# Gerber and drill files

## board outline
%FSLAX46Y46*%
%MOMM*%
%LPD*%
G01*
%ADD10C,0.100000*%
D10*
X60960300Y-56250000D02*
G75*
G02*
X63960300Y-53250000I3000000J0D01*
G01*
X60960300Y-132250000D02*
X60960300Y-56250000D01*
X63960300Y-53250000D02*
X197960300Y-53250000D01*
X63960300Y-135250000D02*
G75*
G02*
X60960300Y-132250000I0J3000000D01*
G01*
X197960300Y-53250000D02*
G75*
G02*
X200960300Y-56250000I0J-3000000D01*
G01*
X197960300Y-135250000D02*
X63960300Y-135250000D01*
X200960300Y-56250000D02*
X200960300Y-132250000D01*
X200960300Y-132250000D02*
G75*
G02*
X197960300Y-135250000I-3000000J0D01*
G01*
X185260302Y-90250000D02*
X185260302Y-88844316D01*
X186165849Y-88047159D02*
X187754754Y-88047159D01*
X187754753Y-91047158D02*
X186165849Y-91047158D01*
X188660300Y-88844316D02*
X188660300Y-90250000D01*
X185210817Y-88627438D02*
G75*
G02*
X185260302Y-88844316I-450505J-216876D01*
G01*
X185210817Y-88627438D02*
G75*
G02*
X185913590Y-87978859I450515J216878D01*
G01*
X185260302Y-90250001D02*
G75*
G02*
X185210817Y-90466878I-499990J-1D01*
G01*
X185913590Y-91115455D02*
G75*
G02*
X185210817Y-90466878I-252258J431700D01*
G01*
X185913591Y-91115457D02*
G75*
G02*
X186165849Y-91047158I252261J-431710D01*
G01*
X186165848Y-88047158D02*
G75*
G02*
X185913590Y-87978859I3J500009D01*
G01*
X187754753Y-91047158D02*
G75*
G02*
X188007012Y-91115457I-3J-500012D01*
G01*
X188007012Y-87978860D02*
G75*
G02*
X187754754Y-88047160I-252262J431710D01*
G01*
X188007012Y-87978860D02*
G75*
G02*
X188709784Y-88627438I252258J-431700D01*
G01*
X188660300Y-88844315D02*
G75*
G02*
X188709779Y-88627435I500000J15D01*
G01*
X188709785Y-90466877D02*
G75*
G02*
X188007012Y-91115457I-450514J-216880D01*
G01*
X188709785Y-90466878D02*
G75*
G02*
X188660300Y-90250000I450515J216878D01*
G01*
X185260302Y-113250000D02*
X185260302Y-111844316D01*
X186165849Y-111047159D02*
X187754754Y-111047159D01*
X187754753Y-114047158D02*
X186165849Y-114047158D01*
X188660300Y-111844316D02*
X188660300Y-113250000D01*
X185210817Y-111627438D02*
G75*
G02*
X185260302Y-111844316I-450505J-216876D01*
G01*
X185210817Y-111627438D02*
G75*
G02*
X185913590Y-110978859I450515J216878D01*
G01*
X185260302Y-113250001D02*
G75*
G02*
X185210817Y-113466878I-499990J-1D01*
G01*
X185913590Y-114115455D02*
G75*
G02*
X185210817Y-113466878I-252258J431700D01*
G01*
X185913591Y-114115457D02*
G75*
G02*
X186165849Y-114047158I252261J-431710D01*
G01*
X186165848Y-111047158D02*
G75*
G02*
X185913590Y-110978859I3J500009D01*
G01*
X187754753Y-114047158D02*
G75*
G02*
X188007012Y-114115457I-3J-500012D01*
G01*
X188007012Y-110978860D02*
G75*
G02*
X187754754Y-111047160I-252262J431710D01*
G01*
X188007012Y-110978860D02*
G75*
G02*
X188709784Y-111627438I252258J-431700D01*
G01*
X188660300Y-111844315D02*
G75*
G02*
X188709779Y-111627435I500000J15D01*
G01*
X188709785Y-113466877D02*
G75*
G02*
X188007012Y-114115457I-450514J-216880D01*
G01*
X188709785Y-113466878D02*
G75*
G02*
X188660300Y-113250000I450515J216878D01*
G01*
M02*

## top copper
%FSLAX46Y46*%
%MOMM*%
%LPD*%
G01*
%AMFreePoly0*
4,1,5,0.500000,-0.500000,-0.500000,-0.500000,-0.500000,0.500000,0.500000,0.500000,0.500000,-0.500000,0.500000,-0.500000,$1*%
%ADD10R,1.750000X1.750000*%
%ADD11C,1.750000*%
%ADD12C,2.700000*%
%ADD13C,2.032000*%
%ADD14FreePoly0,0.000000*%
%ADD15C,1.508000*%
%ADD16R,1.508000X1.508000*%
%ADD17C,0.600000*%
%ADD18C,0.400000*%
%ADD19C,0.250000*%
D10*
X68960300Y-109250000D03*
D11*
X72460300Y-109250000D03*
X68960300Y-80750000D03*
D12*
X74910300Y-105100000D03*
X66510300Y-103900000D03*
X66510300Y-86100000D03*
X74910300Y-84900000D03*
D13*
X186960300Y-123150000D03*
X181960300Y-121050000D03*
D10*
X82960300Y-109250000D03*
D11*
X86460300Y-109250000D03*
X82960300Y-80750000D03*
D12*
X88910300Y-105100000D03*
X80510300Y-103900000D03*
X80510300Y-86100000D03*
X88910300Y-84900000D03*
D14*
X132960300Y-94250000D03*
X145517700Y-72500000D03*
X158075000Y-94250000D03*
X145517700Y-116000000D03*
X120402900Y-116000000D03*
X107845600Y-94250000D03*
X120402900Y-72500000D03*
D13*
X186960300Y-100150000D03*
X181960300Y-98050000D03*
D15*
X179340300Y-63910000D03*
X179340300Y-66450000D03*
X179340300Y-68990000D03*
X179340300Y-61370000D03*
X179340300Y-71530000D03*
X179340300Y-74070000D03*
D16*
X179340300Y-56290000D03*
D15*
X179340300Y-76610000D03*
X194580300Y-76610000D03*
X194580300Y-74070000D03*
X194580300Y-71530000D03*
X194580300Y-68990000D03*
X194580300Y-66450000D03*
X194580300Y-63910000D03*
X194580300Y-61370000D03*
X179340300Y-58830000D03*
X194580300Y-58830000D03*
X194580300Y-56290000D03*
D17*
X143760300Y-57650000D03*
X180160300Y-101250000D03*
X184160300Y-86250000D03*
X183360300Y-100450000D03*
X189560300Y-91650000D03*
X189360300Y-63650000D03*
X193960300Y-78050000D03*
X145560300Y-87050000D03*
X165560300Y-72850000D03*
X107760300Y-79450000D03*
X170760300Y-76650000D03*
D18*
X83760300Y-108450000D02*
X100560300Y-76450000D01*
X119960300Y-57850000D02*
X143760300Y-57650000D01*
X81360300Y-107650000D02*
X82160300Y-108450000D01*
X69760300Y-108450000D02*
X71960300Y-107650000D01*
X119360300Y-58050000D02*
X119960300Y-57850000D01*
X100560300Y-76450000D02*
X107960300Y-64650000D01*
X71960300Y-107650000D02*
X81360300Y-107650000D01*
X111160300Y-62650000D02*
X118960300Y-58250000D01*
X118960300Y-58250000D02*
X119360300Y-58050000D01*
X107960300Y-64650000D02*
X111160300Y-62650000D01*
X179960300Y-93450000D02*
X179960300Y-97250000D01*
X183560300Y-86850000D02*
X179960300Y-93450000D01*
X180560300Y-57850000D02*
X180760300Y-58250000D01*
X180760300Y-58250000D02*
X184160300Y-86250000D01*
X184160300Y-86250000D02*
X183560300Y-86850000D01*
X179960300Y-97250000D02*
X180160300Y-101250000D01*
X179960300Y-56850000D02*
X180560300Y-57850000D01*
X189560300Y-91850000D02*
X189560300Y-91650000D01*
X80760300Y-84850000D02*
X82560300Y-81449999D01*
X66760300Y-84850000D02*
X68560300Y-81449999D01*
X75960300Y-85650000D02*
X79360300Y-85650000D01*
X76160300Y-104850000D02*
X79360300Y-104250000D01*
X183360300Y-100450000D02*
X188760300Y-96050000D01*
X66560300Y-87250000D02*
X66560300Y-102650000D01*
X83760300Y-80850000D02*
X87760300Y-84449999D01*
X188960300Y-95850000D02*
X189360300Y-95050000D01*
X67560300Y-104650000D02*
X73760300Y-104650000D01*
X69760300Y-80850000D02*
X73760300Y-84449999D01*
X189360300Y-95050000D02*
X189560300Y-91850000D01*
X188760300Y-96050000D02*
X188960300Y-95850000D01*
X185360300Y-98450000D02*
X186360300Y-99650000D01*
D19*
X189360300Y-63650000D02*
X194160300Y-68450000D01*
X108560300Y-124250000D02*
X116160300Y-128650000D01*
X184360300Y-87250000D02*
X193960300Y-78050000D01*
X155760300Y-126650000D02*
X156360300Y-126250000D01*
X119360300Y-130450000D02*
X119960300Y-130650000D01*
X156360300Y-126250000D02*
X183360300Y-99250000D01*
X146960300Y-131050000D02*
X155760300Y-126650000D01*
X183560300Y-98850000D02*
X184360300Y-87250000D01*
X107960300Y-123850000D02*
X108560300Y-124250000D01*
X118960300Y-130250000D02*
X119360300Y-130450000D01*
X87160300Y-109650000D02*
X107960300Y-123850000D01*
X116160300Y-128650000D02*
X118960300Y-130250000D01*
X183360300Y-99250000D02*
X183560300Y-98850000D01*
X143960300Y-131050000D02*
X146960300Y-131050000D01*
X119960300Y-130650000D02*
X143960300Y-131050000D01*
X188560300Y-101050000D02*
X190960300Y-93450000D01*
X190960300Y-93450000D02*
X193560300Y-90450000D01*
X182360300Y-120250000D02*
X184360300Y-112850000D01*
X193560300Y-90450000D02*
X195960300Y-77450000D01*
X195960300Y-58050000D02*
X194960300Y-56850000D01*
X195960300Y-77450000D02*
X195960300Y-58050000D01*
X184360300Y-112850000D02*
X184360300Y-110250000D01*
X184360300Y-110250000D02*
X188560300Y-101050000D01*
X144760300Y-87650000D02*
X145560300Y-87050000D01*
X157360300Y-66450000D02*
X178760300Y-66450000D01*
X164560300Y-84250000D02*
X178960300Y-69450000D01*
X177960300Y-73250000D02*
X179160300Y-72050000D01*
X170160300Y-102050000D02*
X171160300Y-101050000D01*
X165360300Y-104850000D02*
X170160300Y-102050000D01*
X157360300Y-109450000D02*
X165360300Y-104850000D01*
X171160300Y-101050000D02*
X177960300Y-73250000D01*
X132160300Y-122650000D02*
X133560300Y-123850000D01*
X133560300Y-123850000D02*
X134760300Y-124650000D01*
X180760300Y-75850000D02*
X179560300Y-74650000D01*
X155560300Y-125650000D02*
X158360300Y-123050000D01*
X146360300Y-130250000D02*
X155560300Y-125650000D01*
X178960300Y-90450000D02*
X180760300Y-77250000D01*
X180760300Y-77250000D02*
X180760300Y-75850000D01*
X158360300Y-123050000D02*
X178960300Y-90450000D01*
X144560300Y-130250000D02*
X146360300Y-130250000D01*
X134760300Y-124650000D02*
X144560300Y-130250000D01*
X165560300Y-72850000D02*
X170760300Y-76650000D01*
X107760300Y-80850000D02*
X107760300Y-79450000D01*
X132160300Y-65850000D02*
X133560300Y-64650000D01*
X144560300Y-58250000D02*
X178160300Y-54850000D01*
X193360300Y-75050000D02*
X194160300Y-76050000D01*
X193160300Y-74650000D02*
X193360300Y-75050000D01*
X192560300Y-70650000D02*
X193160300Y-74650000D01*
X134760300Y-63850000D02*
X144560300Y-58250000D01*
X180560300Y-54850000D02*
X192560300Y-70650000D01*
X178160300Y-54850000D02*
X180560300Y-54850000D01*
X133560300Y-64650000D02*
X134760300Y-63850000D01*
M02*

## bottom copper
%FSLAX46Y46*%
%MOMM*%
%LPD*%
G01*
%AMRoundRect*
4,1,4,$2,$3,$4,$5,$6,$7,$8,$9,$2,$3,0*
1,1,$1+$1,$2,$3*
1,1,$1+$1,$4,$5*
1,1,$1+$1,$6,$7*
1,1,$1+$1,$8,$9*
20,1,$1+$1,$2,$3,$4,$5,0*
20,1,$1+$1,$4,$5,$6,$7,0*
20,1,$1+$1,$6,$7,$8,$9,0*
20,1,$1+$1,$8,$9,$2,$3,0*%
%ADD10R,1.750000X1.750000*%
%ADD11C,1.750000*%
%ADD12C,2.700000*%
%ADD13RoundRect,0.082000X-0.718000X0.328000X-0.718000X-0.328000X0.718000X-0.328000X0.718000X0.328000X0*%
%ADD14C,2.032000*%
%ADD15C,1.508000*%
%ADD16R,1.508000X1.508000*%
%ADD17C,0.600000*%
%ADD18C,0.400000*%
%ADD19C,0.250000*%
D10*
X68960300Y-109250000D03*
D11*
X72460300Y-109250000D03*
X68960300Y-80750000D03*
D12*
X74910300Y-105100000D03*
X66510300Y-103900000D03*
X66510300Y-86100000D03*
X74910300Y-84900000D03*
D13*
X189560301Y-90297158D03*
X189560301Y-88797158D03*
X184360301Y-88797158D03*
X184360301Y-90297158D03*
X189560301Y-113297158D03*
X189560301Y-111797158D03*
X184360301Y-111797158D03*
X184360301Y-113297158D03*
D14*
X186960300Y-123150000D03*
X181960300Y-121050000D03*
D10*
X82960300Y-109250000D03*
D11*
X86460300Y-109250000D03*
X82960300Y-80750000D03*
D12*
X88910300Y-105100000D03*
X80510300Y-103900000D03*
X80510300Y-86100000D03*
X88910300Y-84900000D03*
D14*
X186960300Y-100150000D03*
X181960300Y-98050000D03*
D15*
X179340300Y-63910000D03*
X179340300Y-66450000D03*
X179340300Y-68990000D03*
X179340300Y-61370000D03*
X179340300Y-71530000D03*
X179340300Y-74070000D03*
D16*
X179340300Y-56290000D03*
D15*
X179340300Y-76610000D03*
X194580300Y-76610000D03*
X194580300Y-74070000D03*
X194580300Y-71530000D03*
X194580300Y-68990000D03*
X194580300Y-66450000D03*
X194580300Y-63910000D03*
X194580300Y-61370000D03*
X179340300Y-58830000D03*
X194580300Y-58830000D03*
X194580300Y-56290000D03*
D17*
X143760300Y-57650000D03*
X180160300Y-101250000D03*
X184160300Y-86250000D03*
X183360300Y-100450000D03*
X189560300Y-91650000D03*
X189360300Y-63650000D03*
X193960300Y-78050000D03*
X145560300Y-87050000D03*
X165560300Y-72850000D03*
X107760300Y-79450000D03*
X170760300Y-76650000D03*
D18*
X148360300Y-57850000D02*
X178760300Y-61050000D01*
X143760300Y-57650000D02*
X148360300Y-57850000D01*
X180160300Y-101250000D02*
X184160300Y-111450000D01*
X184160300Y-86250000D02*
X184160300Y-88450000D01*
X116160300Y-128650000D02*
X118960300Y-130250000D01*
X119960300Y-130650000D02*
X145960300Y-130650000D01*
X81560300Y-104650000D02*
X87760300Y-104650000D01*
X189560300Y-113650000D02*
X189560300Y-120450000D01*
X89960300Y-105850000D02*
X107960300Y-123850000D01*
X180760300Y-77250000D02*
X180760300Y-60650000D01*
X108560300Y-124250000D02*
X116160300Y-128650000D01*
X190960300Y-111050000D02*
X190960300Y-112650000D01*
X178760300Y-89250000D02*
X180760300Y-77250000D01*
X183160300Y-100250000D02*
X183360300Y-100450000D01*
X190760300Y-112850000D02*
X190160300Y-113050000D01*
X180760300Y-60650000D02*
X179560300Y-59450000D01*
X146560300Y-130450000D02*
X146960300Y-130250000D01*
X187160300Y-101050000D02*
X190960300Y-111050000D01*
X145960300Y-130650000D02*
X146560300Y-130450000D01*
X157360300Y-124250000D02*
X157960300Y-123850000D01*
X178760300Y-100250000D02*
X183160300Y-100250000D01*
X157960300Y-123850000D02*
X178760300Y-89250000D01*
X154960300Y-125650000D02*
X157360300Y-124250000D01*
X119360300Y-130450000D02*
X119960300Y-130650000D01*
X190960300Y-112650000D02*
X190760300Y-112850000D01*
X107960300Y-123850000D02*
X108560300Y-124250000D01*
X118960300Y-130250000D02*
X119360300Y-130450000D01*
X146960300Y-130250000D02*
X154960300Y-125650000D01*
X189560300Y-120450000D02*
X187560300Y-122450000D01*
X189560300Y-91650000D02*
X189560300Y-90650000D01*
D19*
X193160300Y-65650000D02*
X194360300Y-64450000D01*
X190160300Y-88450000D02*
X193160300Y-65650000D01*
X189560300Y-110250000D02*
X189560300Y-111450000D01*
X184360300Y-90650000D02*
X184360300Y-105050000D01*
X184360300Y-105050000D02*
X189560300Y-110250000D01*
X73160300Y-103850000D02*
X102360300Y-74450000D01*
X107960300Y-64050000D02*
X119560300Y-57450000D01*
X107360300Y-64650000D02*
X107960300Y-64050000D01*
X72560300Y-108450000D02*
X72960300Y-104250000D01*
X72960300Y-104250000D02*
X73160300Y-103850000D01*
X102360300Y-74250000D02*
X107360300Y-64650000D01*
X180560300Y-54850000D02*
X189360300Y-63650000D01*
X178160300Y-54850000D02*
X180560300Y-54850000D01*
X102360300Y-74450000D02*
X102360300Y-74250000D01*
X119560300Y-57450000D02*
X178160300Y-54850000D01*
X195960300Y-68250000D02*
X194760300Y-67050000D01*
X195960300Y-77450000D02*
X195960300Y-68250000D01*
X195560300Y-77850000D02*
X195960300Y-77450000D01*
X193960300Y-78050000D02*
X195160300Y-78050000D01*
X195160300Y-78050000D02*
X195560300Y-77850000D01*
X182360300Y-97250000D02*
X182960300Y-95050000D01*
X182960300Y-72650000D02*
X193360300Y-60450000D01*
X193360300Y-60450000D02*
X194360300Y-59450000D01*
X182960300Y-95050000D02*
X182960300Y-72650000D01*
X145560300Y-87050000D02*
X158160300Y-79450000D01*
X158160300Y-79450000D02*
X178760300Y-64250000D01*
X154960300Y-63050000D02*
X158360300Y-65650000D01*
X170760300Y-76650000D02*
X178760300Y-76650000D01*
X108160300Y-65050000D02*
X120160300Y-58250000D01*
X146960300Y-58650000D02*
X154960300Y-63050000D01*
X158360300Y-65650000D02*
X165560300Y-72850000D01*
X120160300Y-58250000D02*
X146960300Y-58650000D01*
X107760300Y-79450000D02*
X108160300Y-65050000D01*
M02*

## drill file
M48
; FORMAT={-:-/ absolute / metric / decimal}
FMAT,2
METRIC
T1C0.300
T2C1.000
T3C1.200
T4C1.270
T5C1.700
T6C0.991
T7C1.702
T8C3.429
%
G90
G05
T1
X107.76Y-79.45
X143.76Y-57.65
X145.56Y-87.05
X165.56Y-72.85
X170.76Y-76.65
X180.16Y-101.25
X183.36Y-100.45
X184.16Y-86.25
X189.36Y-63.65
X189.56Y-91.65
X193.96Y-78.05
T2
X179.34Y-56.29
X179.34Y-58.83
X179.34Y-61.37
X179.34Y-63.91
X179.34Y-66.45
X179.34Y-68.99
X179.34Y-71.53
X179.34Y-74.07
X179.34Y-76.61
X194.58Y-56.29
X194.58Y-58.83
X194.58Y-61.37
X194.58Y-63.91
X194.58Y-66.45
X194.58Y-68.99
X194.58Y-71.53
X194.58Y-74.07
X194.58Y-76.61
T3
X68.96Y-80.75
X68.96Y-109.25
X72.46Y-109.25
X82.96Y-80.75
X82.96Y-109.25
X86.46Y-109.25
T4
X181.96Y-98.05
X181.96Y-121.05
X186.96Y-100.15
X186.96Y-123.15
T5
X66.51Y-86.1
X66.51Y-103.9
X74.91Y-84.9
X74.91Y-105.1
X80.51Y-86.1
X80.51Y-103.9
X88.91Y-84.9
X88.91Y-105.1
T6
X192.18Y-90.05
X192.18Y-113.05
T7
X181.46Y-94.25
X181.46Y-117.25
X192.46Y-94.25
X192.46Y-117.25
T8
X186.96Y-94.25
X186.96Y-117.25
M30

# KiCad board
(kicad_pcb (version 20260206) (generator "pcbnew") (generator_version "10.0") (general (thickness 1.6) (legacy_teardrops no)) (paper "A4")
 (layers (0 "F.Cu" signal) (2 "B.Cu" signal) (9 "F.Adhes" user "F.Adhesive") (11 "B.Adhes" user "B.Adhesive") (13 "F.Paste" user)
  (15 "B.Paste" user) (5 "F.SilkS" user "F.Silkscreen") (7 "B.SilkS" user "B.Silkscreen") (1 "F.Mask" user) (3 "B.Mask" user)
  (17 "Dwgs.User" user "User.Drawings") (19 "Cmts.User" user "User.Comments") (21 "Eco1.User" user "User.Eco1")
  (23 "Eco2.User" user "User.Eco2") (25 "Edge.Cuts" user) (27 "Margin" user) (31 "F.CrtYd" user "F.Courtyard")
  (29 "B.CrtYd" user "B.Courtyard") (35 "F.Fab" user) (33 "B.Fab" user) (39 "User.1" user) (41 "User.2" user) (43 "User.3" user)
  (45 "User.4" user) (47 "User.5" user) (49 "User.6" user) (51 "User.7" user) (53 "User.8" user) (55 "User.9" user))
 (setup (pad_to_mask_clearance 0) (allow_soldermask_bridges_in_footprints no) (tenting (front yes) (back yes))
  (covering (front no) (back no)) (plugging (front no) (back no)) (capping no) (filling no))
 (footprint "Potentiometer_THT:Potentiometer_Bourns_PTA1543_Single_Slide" (layer "F.Cu") (at 68.9603 109.25 90)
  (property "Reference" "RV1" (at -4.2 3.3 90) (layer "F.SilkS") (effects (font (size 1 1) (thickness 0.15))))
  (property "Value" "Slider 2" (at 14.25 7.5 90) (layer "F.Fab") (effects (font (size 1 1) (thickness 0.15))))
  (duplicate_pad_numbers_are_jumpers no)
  (pad "1" thru_hole rect (at 0 0 90) (size 1.75 1.75) (drill 1.2) (layers "*.Cu" "*.Mask") (remove_unused_layers no) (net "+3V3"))
  (pad "2" thru_hole circle (at 0 3.5 90) (size 1.75 1.75) (drill 1.2) (layers "*.Cu" "*.Mask") (remove_unused_layers no) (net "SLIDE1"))
  (pad "3" thru_hole circle (at 28.5 0 90) (size 1.75 1.75) (drill 1.2) (layers "*.Cu" "*.Mask") (remove_unused_layers no) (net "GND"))
  (pad "MP" thru_hole circle (at 4.15 5.95 90) (size 2.7 2.7) (drill 1.7) (layers "*.Cu" "*.Mask") (remove_unused_layers no) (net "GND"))
  (pad "MP" thru_hole circle (at 5.35 -2.45 90) (size 2.7 2.7) (drill 1.7) (layers "*.Cu" "*.Mask") (remove_unused_layers no) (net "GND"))
  (pad "MP" thru_hole circle (at 23.15 -2.45 90) (size 2.7 2.7) (drill 1.7) (layers "*.Cu" "*.Mask") (remove_unused_layers no) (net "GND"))
  (pad "MP" thru_hole circle (at 24.35 5.95 90) (size 2.7 2.7) (drill 1.7) (layers "*.Cu" "*.Mask") (remove_unused_layers no) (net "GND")))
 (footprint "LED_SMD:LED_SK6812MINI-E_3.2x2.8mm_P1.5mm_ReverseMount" (layer "F.Cu") (at 186.9603 89.65)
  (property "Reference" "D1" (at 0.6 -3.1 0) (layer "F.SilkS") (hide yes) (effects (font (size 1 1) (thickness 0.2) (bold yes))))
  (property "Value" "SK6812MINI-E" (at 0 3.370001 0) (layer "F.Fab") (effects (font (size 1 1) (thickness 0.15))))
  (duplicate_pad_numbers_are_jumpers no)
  (fp_line (start -1.699998 0.6) (end -1.699998 -0.805684) (stroke (width 0.1) (type solid)) (layer "Edge.Cuts"))
  (fp_line (start -0.794451 -1.602841) (end 0.794454 -1.602841) (stroke (width 0.1) (type solid)) (layer "Edge.Cuts"))
  (fp_line (start 0.794453 1.397158) (end -0.794451 1.397158) (stroke (width 0.1) (type solid)) (layer "Edge.Cuts"))
  (fp_line (start 1.7 -0.805684) (end 1.7 0.6) (stroke (width 0.1) (type solid)) (layer "Edge.Cuts"))
  (fp_arc (start -1.749483 -1.022562) (mid -1.712526 -0.91691) (end -1.699998 -0.805684) (stroke (width 0.1) (type solid))
   (layer "Edge.Cuts"))
  (fp_arc (start -1.749483 -1.022562) (mid -1.63807 -1.606877) (end -1.04671 -1.671141) (stroke (width 0.1) (type solid))
   (layer "Edge.Cuts"))
  (fp_arc (start -1.699998 0.600001) (mid -1.712526 0.711226) (end -1.749483 0.816878) (stroke (width 0.1) (type solid)) (layer "Edge.Cuts"))
  (fp_arc (start -1.04671 1.465455) (mid -1.638069 1.401192) (end -1.749483 0.816878) (stroke (width 0.1) (type solid)) (layer "Edge.Cuts"))
  (fp_arc (start -1.046709 1.465457) (mid -0.925121 1.414535) (end -0.794451 1.397158) (stroke (width 0.1) (type solid)) (layer "Edge.Cuts"))
  (fp_arc (start -0.794452 -1.602842) (mid -0.925122 -1.620219) (end -1.04671 -1.671141) (stroke (width 0.1) (type solid))
   (layer "Edge.Cuts"))
  (fp_arc (start 0.794453 1.397158) (mid 0.925124 1.414535) (end 1.046712 1.465457) (stroke (width 0.1) (type solid)) (layer "Edge.Cuts"))
  (fp_arc (start 1.046712 -1.67114) (mid 0.925124 -1.620218) (end 0.794454 -1.602841) (stroke (width 0.1) (type solid)) (layer "Edge.Cuts"))
  (fp_arc (start 1.046712 -1.67114) (mid 1.638072 -1.606876) (end 1.749485 -1.022562) (stroke (width 0.1) (type solid)) (layer "Edge.Cuts"))
  (fp_arc (start 1.7 -0.805685) (mid 1.712528 -0.91691) (end 1.749485 -1.022562) (stroke (width 0.1) (type solid)) (layer "Edge.Cuts"))
  (fp_arc (start 1.749485 0.816877) (mid 1.638073 1.401193) (end 1.046712 1.465457) (stroke (width 0.1) (type solid)) (layer "Edge.Cuts"))
  (fp_arc (start 1.749485 0.816878) (mid 1.712528 0.711226) (end 1.7 0.6) (stroke (width 0.1) (type solid)) (layer "Edge.Cuts"))
  (pad "1" smd roundrect (at 2.600001 0.647158 270) (size 0.82 1.6) (layers "B.Cu" "B.Mask" "B.Paste") (roundrect_rratio 0.1) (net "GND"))
  (pad "2" smd roundrect (at 2.600001 -0.852842 270) (size 0.82 1.6) (layers "B.Cu" "B.Mask" "B.Paste") (roundrect_rratio 0.1) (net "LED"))
  (pad "3" smd roundrect (at -2.599999 -0.852842 270) (size 0.82 1.6) (layers "B.Cu" "B.Mask" "B.Paste") (roundrect_rratio 0.1) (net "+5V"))
  (pad "4" smd roundrect (at -2.599999 0.647158 270) (size 0.82 1.6) (layers "B.Cu" "B.Mask" "B.Paste") (roundrect_rratio 0.1)
   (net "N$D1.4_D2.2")))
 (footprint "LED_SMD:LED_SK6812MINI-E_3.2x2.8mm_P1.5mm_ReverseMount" (layer "F.Cu") (at 186.9603 112.65)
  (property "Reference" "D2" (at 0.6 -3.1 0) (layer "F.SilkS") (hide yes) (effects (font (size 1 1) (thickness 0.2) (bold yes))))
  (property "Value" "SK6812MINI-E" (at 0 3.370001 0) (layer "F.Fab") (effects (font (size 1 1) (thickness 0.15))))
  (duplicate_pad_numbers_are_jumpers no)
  (fp_line (start -1.699998 0.6) (end -1.699998 -0.805684) (stroke (width 0.1) (type solid)) (layer "Edge.Cuts"))
  (fp_line (start -0.794451 -1.602841) (end 0.794454 -1.602841) (stroke (width 0.1) (type solid)) (layer "Edge.Cuts"))
  (fp_line (start 0.794453 1.397158) (end -0.794451 1.397158) (stroke (width 0.1) (type solid)) (layer "Edge.Cuts"))
  (fp_line (start 1.7 -0.805684) (end 1.7 0.6) (stroke (width 0.1) (type solid)) (layer "Edge.Cuts"))
  (fp_arc (start -1.749483 -1.022562) (mid -1.712526 -0.91691) (end -1.699998 -0.805684) (stroke (width 0.1) (type solid))
   (layer "Edge.Cuts"))
  (fp_arc (start -1.749483 -1.022562) (mid -1.63807 -1.606877) (end -1.04671 -1.671141) (stroke (width 0.1) (type solid))
   (layer "Edge.Cuts"))
  (fp_arc (start -1.699998 0.600001) (mid -1.712526 0.711226) (end -1.749483 0.816878) (stroke (width 0.1) (type solid)) (layer "Edge.Cuts"))
  (fp_arc (start -1.04671 1.465455) (mid -1.638069 1.401192) (end -1.749483 0.816878) (stroke (width 0.1) (type solid)) (layer "Edge.Cuts"))
  (fp_arc (start -1.046709 1.465457) (mid -0.925121 1.414535) (end -0.794451 1.397158) (stroke (width 0.1) (type solid)) (layer "Edge.Cuts"))
  (fp_arc (start -0.794452 -1.602842) (mid -0.925122 -1.620219) (end -1.04671 -1.671141) (stroke (width 0.1) (type solid))
   (layer "Edge.Cuts"))
  (fp_arc (start 0.794453 1.397158) (mid 0.925124 1.414535) (end 1.046712 1.465457) (stroke (width 0.1) (type solid)) (layer "Edge.Cuts"))
  (fp_arc (start 1.046712 -1.67114) (mid 0.925124 -1.620218) (end 0.794454 -1.602841) (stroke (width 0.1) (type solid)) (layer "Edge.Cuts"))
  (fp_arc (start 1.046712 -1.67114) (mid 1.638072 -1.606876) (end 1.749485 -1.022562) (stroke (width 0.1) (type solid)) (layer "Edge.Cuts"))
  (fp_arc (start 1.7 -0.805685) (mid 1.712528 -0.91691) (end 1.749485 -1.022562) (stroke (width 0.1) (type solid)) (layer "Edge.Cuts"))
  (fp_arc (start 1.749485 0.816877) (mid 1.638073 1.401193) (end 1.046712 1.465457) (stroke (width 0.1) (type solid)) (layer "Edge.Cuts"))
  (fp_arc (start 1.749485 0.816878) (mid 1.712528 0.711226) (end 1.7 0.6) (stroke (width 0.1) (type solid)) (layer "Edge.Cuts"))
  (pad "1" smd roundrect (at 2.600001 0.647158 270) (size 0.82 1.6) (layers "B.Cu" "B.Mask" "B.Paste") (roundrect_rratio 0.1) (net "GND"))
  (pad "2" smd roundrect (at 2.600001 -0.852842 270) (size 0.82 1.6) (layers "B.Cu" "B.Mask" "B.Paste") (roundrect_rratio 0.1)
   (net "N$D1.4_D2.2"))
  (pad "3" smd roundrect (at -2.599999 -0.852842 270) (size 0.82 1.6) (layers "B.Cu" "B.Mask" "B.Paste") (roundrect_rratio 0.1) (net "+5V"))
  (pad "4" smd roundrect (at -2.599999 0.647158 270) (size 0.82 1.6) (layers "B.Cu" "B.Mask" "B.Paste") (roundrect_rratio 0.1)))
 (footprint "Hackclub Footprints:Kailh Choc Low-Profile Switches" (layer "F.Cu") (at 186.9603 117.25)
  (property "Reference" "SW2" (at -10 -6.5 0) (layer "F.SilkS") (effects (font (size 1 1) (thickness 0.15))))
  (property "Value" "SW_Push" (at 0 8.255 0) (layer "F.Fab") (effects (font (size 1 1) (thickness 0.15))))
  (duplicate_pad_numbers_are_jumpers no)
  (pad "" np_thru_hole circle (at -5.5 0) (size 1.7018 1.7018) (drill 1.7018) (layers "*.Cu" "*.Mask"))
  (pad "" np_thru_hole circle (at 0 0) (size 3.429 3.429) (drill 3.429) (layers "*.Cu" "*.Mask"))
  (pad "" np_thru_hole circle (at 5.22 -4.2) (size 0.9906 0.9906) (drill 0.9906) (layers "*.Cu" "*.Mask"))
  (pad "" np_thru_hole circle (at 5.5 0) (size 1.7018 1.7018) (drill 1.7018) (layers "*.Cu" "*.Mask"))
  (pad "1" thru_hole circle (at 0 5.9) (size 2.032 2.032) (drill 1.27) (layers "*.Cu" "*.Mask") (remove_unused_layers no) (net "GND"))
  (pad "2" thru_hole circle (at -5 3.8) (size 2.032 2.032) (drill 1.27) (layers "*.Cu" "*.Mask") (remove_unused_layers no) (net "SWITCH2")))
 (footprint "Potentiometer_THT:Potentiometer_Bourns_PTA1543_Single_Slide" (layer "F.Cu") (at 82.9603 109.25 90)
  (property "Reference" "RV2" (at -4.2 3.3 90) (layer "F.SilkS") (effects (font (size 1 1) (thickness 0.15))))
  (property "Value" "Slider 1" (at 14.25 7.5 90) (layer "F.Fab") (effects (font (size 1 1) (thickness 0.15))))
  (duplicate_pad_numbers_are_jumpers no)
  (pad "1" thru_hole rect (at 0 0 90) (size 1.75 1.75) (drill 1.2) (layers "*.Cu" "*.Mask") (remove_unused_layers no) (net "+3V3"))
  (pad "2" thru_hole circle (at 0 3.5 90) (size 1.75 1.75) (drill 1.2) (layers "*.Cu" "*.Mask") (remove_unused_layers no) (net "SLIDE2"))
  (pad "3" thru_hole circle (at 28.5 0 90) (size 1.75 1.75) (drill 1.2) (layers "*.Cu" "*.Mask") (remove_unused_layers no) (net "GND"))
  (pad "MP" thru_hole circle (at 4.15 5.95 90) (size 2.7 2.7) (drill 1.7) (layers "*.Cu" "*.Mask") (remove_unused_layers no) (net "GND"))
  (pad "MP" thru_hole circle (at 5.35 -2.45 90) (size 2.7 2.7) (drill 1.7) (layers "*.Cu" "*.Mask") (remove_unused_layers no) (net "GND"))
  (pad "MP" thru_hole circle (at 23.15 -2.45 90) (size 2.7 2.7) (drill 1.7) (layers "*.Cu" "*.Mask") (remove_unused_layers no) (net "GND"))
  (pad "MP" thru_hole circle (at 24.35 5.95 90) (size 2.7 2.7) (drill 1.7) (layers "*.Cu" "*.Mask") (remove_unused_layers no) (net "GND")))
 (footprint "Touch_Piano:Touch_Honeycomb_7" (layer "F.Cu") (at 132.9603 94.25)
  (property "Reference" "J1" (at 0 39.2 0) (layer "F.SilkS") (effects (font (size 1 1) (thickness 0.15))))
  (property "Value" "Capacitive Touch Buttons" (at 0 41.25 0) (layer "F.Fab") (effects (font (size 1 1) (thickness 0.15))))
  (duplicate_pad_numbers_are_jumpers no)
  (pad "1" smd custom (at 0 0) (size 1 1) (layers "F.Cu") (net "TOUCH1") (zone_connect 0) (options (clearance outline) (anchor rect))
   (primitives))
  (pad "2" smd custom (at 12.5574 -21.75) (size 1 1) (layers "F.Cu") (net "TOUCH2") (zone_connect 0)
   (options (clearance outline) (anchor rect)) (primitives))
  (pad "3" smd custom (at 25.1147 0) (size 1 1) (layers "F.Cu") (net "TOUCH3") (zone_connect 0) (options (clearance outline) (anchor rect))
   (primitives))
  (pad "4" smd custom (at 12.5574 21.75) (size 1 1) (layers "F.Cu") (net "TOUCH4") (zone_connect 0)
   (options (clearance outline) (anchor rect)) (primitives))
  (pad "5" smd custom (at -12.5574 21.75) (size 1 1) (layers "F.Cu") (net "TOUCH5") (zone_connect 0)
   (options (clearance outline) (anchor rect)) (primitives))
  (pad "6" smd custom (at -25.1147 0) (size 1 1) (layers "F.Cu") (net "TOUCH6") (zone_connect 0) (options (clearance outline) (anchor rect))
   (primitives))
  (pad "7" smd custom (at -12.5574 -21.75) (size 1 1) (layers "F.Cu") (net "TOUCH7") (zone_connect 0)
   (options (clearance outline) (anchor rect)) (primitives)))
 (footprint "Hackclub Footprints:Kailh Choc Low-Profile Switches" (layer "F.Cu") (at 186.9603 94.25)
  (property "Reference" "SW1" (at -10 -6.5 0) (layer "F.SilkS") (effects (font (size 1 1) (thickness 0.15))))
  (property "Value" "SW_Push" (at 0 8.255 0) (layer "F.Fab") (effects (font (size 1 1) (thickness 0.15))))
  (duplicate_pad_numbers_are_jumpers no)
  (pad "" np_thru_hole circle (at -5.5 0) (size 1.7018 1.7018) (drill 1.7018) (layers "*.Cu" "*.Mask"))
  (pad "" np_thru_hole circle (at 0 0) (size 3.429 3.429) (drill 3.429) (layers "*.Cu" "*.Mask"))
  (pad "" np_thru_hole circle (at 5.22 -4.2) (size 0.9906 0.9906) (drill 0.9906) (layers "*.Cu" "*.Mask"))
  (pad "" np_thru_hole circle (at 5.5 0) (size 1.7018 1.7018) (drill 1.7018) (layers "*.Cu" "*.Mask"))
  (pad "1" thru_hole circle (at 0 5.9) (size 2.032 2.032) (drill 1.27) (layers "*.Cu" "*.Mask") (remove_unused_layers no) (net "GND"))
  (pad "2" thru_hole circle (at -5 3.8) (size 2.032 2.032) (drill 1.27) (layers "*.Cu" "*.Mask") (remove_unused_layers no) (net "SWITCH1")))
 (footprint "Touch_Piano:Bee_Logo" (layer "F.Cu") (at 77.4603 124.75)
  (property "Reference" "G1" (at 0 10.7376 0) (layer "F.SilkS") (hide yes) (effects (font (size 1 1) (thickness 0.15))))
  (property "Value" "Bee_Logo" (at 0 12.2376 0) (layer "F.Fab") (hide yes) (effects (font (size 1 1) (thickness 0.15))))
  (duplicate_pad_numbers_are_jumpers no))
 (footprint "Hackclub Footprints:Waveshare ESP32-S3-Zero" (layer "F.Cu") (at 186.9603 66.45)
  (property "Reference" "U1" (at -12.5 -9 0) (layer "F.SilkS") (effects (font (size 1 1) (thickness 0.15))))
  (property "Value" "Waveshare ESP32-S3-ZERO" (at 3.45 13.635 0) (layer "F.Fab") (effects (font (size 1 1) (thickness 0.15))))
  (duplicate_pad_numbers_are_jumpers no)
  (pad "1" thru_hole circle (at -7.62 -2.54) (size 1.508 1.508) (drill 1) (layers "*.Cu" "*.Mask") (remove_unused_layers no) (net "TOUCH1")
   (solder_mask_margin 0.102))
  (pad "2" thru_hole circle (at -7.62 0) (size 1.508 1.508) (drill 1) (layers "*.Cu" "*.Mask") (remove_unused_layers no) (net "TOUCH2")
   (solder_mask_margin 0.102))
  (pad "3" thru_hole circle (at -7.62 2.54) (size 1.508 1.508) (drill 1) (layers "*.Cu" "*.Mask") (remove_unused_layers no) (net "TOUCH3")
   (solder_mask_margin 0.102))
  (pad "3V3" thru_hole circle (at -7.62 -5.08) (size 1.508 1.508) (drill 1) (layers "*.Cu" "*.Mask") (remove_unused_layers no) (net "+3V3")
   (solder_mask_margin 0.102))
  (pad "4" thru_hole circle (at -7.62 5.08) (size 1.508 1.508) (drill 1) (layers "*.Cu" "*.Mask") (remove_unused_layers no) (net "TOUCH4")
   (solder_mask_margin 0.102))
  (pad "5" thru_hole circle (at -7.62 7.62) (size 1.508 1.508) (drill 1) (layers "*.Cu" "*.Mask") (remove_unused_layers no) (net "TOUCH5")
   (solder_mask_margin 0.102))
  (pad "5V" thru_hole rect (at -7.62 -10.16) (size 1.508 1.508) (drill 1) (layers "*.Cu" "*.Mask") (remove_unused_layers no) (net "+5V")
   (solder_mask_margin 0.102))
  (pad "6" thru_hole circle (at -7.62 10.16) (size 1.508 1.508) (drill 1) (layers "*.Cu" "*.Mask") (remove_unused_layers no) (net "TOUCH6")
   (solder_mask_margin 0.102))
  (pad "7" thru_hole circle (at 7.62 10.16) (size 1.508 1.508) (drill 1) (layers "*.Cu" "*.Mask") (remove_unused_layers no) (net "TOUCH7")
   (solder_mask_margin 0.102))
  (pad "8" thru_hole circle (at 7.62 7.62) (size 1.508 1.508) (drill 1) (layers "*.Cu" "*.Mask") (remove_unused_layers no)
   (solder_mask_margin 0.102))
  (pad "9" thru_hole circle (at 7.62 5.08) (size 1.508 1.508) (drill 1) (layers "*.Cu" "*.Mask") (remove_unused_layers no)
   (solder_mask_margin 0.102))
  (pad "10" thru_hole circle (at 7.62 2.54) (size 1.508 1.508) (drill 1) (layers "*.Cu" "*.Mask") (remove_unused_layers no) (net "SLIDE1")
   (solder_mask_margin 0.102))
  (pad "11" thru_hole circle (at 7.62 0) (size 1.508 1.508) (drill 1) (layers "*.Cu" "*.Mask") (remove_unused_layers no) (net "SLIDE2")
   (solder_mask_margin 0.102))
  (pad "12" thru_hole circle (at 7.62 -2.54) (size 1.508 1.508) (drill 1) (layers "*.Cu" "*.Mask") (remove_unused_layers no) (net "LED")
   (solder_mask_margin 0.102))
  (pad "13" thru_hole circle (at 7.62 -5.08) (size 1.508 1.508) (drill 1) (layers "*.Cu" "*.Mask") (remove_unused_layers no)
   (solder_mask_margin 0.102))
  (pad "GND" thru_hole circle (at -7.62 -7.62) (size 1.508 1.508) (drill 1) (layers "*.Cu" "*.Mask") (remove_unused_layers no) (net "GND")
   (solder_mask_margin 0.102))
  (pad "RX" thru_hole circle (at 7.62 -7.62) (size 1.508 1.508) (drill 1) (layers "*.Cu" "*.Mask") (remove_unused_layers no) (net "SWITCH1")
   (solder_mask_margin 0.102))
  (pad "TX" thru_hole circle (at 7.62 -10.16) (size 1.508 1.508) (drill 1) (layers "*.Cu" "*.Mask") (remove_unused_layers no)
   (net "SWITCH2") (solder_mask_margin 0.102)))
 (gr_arc (start 60.9603 56.25) (mid 61.83898 54.12868) (end 63.9603 53.25) (stroke (width 0.1) (type default)) (layer "Edge.Cuts"))
 (gr_line (start 60.9603 132.25) (end 60.9603 56.25) (stroke (width 0.1) (type default)) (layer "Edge.Cuts"))
 (gr_line (start 63.9603 53.25) (end 197.9603 53.25) (stroke (width 0.1) (type default)) (layer "Edge.Cuts"))
 (gr_arc (start 63.9603 135.25) (mid 61.83898 134.37132) (end 60.9603 132.25) (stroke (width 0.1) (type default)) (layer "Edge.Cuts"))
 (gr_arc (start 197.9603 53.25) (mid 200.08162 54.12868) (end 200.9603 56.25) (stroke (width 0.1) (type default)) (layer "Edge.Cuts"))
 (gr_line (start 197.9603 135.25) (end 63.9603 135.25) (stroke (width 0.1) (type default)) (layer "Edge.Cuts"))
 (gr_line (start 200.9603 56.25) (end 200.9603 132.25) (stroke (width 0.1) (type default)) (layer "Edge.Cuts"))
 (gr_arc (start 200.9603 132.25) (mid 200.08162 134.37132) (end 197.9603 135.25) (stroke (width 0.1) (type default)) (layer "Edge.Cuts"))
 (segment (start 83.7603 108.45) (end 100.5603 76.45) (width 0.4) (layer "F.Cu") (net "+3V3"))
 (segment (start 119.9603 57.85) (end 143.7603 57.65) (width 0.4) (layer "F.Cu") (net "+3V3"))
 (segment (start 81.3603 107.65) (end 82.1603 108.45) (width 0.4) (layer "F.Cu") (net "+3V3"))
 (segment (start 69.7603 108.45) (end 71.9603 107.65) (width 0.4) (layer "F.Cu") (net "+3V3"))
 (segment (start 119.3603 58.05) (end 119.9603 57.85) (width 0.4) (layer "F.Cu") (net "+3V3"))
 (segment (start 100.5603 76.45) (end 107.9603 64.65) (width 0.4) (layer "F.Cu") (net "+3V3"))
 (segment (start 71.9603 107.65) (end 81.3603 107.65) (width 0.4) (layer "F.Cu") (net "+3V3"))
 (segment (start 111.1603 62.65) (end 118.9603 58.25) (width 0.4) (layer "F.Cu") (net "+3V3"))
 (segment (start 118.9603 58.25) (end 119.3603 58.05) (width 0.4) (layer "F.Cu") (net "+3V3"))
 (segment (start 107.9603 64.65) (end 111.1603 62.65) (width 0.4) (layer "F.Cu") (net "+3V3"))
 (via (at 143.7603 57.65) (size 0.6) (drill 0.3) (layers "F.Cu" "B.Cu") (capping no) (covering (front no) (back no))
  (plugging (front no) (back no)) (filling no) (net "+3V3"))
 (segment (start 148.3603 57.85) (end 178.7603 61.05) (width 0.4) (layer "B.Cu") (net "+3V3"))
 (segment (start 143.7603 57.65) (end 148.3603 57.85) (width 0.4) (layer "B.Cu") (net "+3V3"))
 (segment (start 179.9603 93.45) (end 179.9603 97.25) (width 0.4) (layer "F.Cu") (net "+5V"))
 (segment (start 183.5603 86.85) (end 179.9603 93.45) (width 0.4) (layer "F.Cu") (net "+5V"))
 (segment (start 180.5603 57.85) (end 180.7603 58.25) (width 0.4) (layer "F.Cu") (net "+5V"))
 (segment (start 180.7603 58.25) (end 184.1603 86.25) (width 0.4) (layer "F.Cu") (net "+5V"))
 (segment (start 184.1603 86.25) (end 183.5603 86.85) (width 0.4) (layer "F.Cu") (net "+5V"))
 (segment (start 179.9603 97.25) (end 180.1603 101.25) (width 0.4) (layer "F.Cu") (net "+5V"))
 (segment (start 179.9603 56.85) (end 180.5603 57.85) (width 0.4) (layer "F.Cu") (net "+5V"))
 (via (at 180.1603 101.25) (size 0.6) (drill 0.3) (layers "F.Cu" "B.Cu") (capping no) (covering (front no) (back no))
  (plugging (front no) (back no)) (filling no) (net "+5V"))
 (via (at 184.1603 86.25) (size 0.6) (drill 0.3) (layers "F.Cu" "B.Cu") (capping no) (covering (front no) (back no))
  (plugging (front no) (back no)) (filling no) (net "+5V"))
 (segment (start 180.1603 101.25) (end 184.1603 111.45) (width 0.4) (layer "B.Cu") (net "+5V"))
 (segment (start 184.1603 86.25) (end 184.1603 88.45) (width 0.4) (layer "B.Cu") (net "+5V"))
 (segment (start 189.5603 91.85) (end 189.5603 91.65) (width 0.4) (layer "F.Cu") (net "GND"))
 (segment (start 80.7603 84.85) (end 82.5603 81.449999) (width 0.4) (layer "F.Cu") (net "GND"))
 (segment (start 66.7603 84.85) (end 68.5603 81.449999) (width 0.4) (layer "F.Cu") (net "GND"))
 (segment (start 75.9603 85.65) (end 79.3603 85.65) (width 0.4) (layer "F.Cu") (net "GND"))
 (segment (start 76.1603 104.85) (end 79.3603 104.25) (width 0.4) (layer "F.Cu") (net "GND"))
 (segment (start 183.3603 100.45) (end 188.7603 96.05) (width 0.4) (layer "F.Cu") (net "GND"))
 (segment (start 66.5603 87.25) (end 66.5603 102.65) (width 0.4) (layer "F.Cu") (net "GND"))
 (segment (start 83.7603 80.85) (end 87.7603 84.449999) (width 0.4) (layer "F.Cu") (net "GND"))
 (segment (start 188.9603 95.85) (end 189.3603 95.05) (width 0.4) (layer "F.Cu") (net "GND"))
 (segment (start 67.5603 104.65) (end 73.7603 104.65) (width 0.4) (layer "F.Cu") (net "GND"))
 (segment (start 69.7603 80.85) (end 73.7603 84.449999) (width 0.4) (layer "F.Cu") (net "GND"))
 (segment (start 189.3603 95.05) (end 189.5603 91.85) (width 0.4) (layer "F.Cu") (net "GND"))
 (segment (start 188.7603 96.05) (end 188.9603 95.85) (width 0.4) (layer "F.Cu") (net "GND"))
 (segment (start 185.3603 98.45) (end 186.3603 99.65) (width 0.4) (layer "F.Cu") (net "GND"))
 (via (at 183.3603 100.45) (size 0.6) (drill 0.3) (layers "F.Cu" "B.Cu") (capping no) (covering (front no) (back no))
  (plugging (front no) (back no)) (filling no) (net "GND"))
 (via (at 189.5603 91.65) (size 0.6) (drill 0.3) (layers "F.Cu" "B.Cu") (capping no) (covering (front no) (back no))
  (plugging (front no) (back no)) (filling no) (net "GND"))
 (segment (start 116.1603 128.65) (end 118.9603 130.25) (width 0.4) (layer "B.Cu") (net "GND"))
 (segment (start 119.9603 130.65) (end 145.9603 130.65) (width 0.4) (layer "B.Cu") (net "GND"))
 (segment (start 81.5603 104.65) (end 87.7603 104.65) (width 0.4) (layer "B.Cu") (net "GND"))
 (segment (start 189.5603 113.65) (end 189.5603 120.45) (width 0.4) (layer "B.Cu") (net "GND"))
 (segment (start 89.9603 105.85) (end 107.9603 123.85) (width 0.4) (layer "B.Cu") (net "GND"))
 (segment (start 180.7603 77.25) (end 180.7603 60.65) (width 0.4) (layer "B.Cu") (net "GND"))
 (segment (start 108.5603 124.25) (end 116.1603 128.65) (width 0.4) (layer "B.Cu") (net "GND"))
 (segment (start 190.9603 111.05) (end 190.9603 112.65) (width 0.4) (layer "B.Cu") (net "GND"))
 (segment (start 178.7603 89.25) (end 180.7603 77.25) (width 0.4) (layer "B.Cu") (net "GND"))
 (segment (start 183.1603 100.25) (end 183.3603 100.45) (width 0.4) (layer "B.Cu") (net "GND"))
 (segment (start 190.7603 112.85) (end 190.1603 113.05) (width 0.4) (layer "B.Cu") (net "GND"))
 (segment (start 180.7603 60.65) (end 179.5603 59.45) (width 0.4) (layer "B.Cu") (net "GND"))
 (segment (start 146.5603 130.45) (end 146.9603 130.25) (width 0.4) (layer "B.Cu") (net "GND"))
 (segment (start 187.1603 101.05) (end 190.9603 111.05) (width 0.4) (layer "B.Cu") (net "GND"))
 (segment (start 145.9603 130.65) (end 146.5603 130.45) (width 0.4) (layer "B.Cu") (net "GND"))
 (segment (start 157.3603 124.25) (end 157.9603 123.85) (width 0.4) (layer "B.Cu") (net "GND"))
 (segment (start 178.7603 100.25) (end 183.1603 100.25) (width 0.4) (layer "B.Cu") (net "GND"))
 (segment (start 157.9603 123.85) (end 178.7603 89.25) (width 0.4) (layer "B.Cu") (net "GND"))
 (segment (start 154.9603 125.65) (end 157.3603 124.25) (width 0.4) (layer "B.Cu") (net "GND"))
 (segment (start 119.3603 130.45) (end 119.9603 130.65) (width 0.4) (layer "B.Cu") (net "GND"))
 (segment (start 190.9603 112.65) (end 190.7603 112.85) (width 0.4) (layer "B.Cu") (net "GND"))
 (segment (start 107.9603 123.85) (end 108.5603 124.25) (width 0.4) (layer "B.Cu") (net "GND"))
 (segment (start 118.9603 130.25) (end 119.3603 130.45) (width 0.4) (layer "B.Cu") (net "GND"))
 (segment (start 146.9603 130.25) (end 154.9603 125.65) (width 0.4) (layer "B.Cu") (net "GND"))
 (segment (start 189.5603 120.45) (end 187.5603 122.45) (width 0.4) (layer "B.Cu") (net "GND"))
 (segment (start 189.5603 91.65) (end 189.5603 90.65) (width 0.4) (layer "B.Cu") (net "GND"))
 (segment (start 193.1603 65.65) (end 194.3603 64.45) (width 0.25) (layer "B.Cu") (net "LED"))
 (segment (start 190.1603 88.45) (end 193.1603 65.65) (width 0.25) (layer "B.Cu") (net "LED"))
 (segment (start 189.5603 110.25) (end 189.5603 111.45) (width 0.25) (layer "B.Cu") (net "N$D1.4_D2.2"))
 (segment (start 184.3603 90.65) (end 184.3603 105.05) (width 0.25) (layer "B.Cu") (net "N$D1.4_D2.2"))
 (segment (start 184.3603 105.05) (end 189.5603 110.25) (width 0.25) (layer "B.Cu") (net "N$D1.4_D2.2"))
 (segment (start 189.3603 63.65) (end 194.1603 68.45) (width 0.25) (layer "F.Cu") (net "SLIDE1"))
 (via (at 189.3603 63.65) (size 0.6) (drill 0.3) (layers "F.Cu" "B.Cu") (capping no) (covering (front no) (back no))
  (plugging (front no) (back no)) (filling no) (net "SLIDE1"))
 (segment (start 73.1603 103.85) (end 102.3603 74.45) (width 0.25) (layer "B.Cu") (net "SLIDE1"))
 (segment (start 107.9603 64.05) (end 119.5603 57.45) (width 0.25) (layer "B.Cu") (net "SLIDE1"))
 (segment (start 107.3603 64.65) (end 107.9603 64.05) (width 0.25) (layer "B.Cu") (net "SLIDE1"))
 (segment (start 72.5603 108.45) (end 72.9603 104.25) (width 0.25) (layer "B.Cu") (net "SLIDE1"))
 (segment (start 72.9603 104.25) (end 73.1603 103.85) (width 0.25) (layer "B.Cu") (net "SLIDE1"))
 (segment (start 102.3603 74.25) (end 107.3603 64.65) (width 0.25) (layer "B.Cu") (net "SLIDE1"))
 (segment (start 180.5603 54.85) (end 189.3603 63.65) (width 0.25) (layer "B.Cu") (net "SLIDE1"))
 (segment (start 178.1603 54.85) (end 180.5603 54.85) (width 0.25) (layer "B.Cu") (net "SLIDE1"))
 (segment (start 102.3603 74.45) (end 102.3603 74.25) (width 0.25) (layer "B.Cu") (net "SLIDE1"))
 (segment (start 119.5603 57.45) (end 178.1603 54.85) (width 0.25) (layer "B.Cu") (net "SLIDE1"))
 (segment (start 108.5603 124.25) (end 116.1603 128.65) (width 0.25) (layer "F.Cu") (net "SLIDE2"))
 (segment (start 184.3603 87.25) (end 193.9603 78.05) (width 0.25) (layer "F.Cu") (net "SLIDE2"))
 (segment (start 155.7603 126.65) (end 156.3603 126.25) (width 0.25) (layer "F.Cu") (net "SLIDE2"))
 (segment (start 119.3603 130.45) (end 119.9603 130.65) (width 0.25) (layer "F.Cu") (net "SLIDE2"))
 (segment (start 156.3603 126.25) (end 183.3603 99.25) (width 0.25) (layer "F.Cu") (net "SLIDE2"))
 (segment (start 146.9603 131.05) (end 155.7603 126.65) (width 0.25) (layer "F.Cu") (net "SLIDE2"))
 (segment (start 183.5603 98.85) (end 184.3603 87.25) (width 0.25) (layer "F.Cu") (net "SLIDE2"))
 (segment (start 107.9603 123.85) (end 108.5603 124.25) (width 0.25) (layer "F.Cu") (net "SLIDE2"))
 (segment (start 118.9603 130.25) (end 119.3603 130.45) (width 0.25) (layer "F.Cu") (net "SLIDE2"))
 (segment (start 87.1603 109.65) (end 107.9603 123.85) (width 0.25) (layer "F.Cu") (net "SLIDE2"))
 (segment (start 116.1603 128.65) (end 118.9603 130.25) (width 0.25) (layer "F.Cu") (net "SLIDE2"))
 (segment (start 183.3603 99.25) (end 183.5603 98.85) (width 0.25) (layer "F.Cu") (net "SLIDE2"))
 (segment (start 143.9603 131.05) (end 146.9603 131.05) (width 0.25) (layer "F.Cu") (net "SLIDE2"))
 (segment (start 119.9603 130.65) (end 143.9603 131.05) (width 0.25) (layer "F.Cu") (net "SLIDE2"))
 (via (at 193.9603 78.05) (size 0.6) (drill 0.3) (layers "F.Cu" "B.Cu") (capping no) (covering (front no) (back no))
  (plugging (front no) (back no)) (filling no) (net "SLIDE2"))
 (segment (start 195.9603 68.25) (end 194.7603 67.05) (width 0.25) (layer "B.Cu") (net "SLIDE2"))
 (segment (start 195.9603 77.45) (end 195.9603 68.25) (width 0.25) (layer "B.Cu") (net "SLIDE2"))
 (segment (start 195.5603 77.85) (end 195.9603 77.45) (width 0.25) (layer "B.Cu") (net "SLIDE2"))
 (segment (start 193.9603 78.05) (end 195.1603 78.05) (width 0.25) (layer "B.Cu") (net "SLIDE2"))
 (segment (start 195.1603 78.05) (end 195.5603 77.85) (width 0.25) (layer "B.Cu") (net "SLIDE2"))
 (segment (start 182.3603 97.25) (end 182.9603 95.05) (width 0.25) (layer "B.Cu") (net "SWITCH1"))
 (segment (start 182.9603 72.65) (end 193.3603 60.45) (width 0.25) (layer "B.Cu") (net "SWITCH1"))
 (segment (start 193.3603 60.45) (end 194.3603 59.45) (width 0.25) (layer "B.Cu") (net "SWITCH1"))
 (segment (start 182.9603 95.05) (end 182.9603 72.65) (width 0.25) (layer "B.Cu") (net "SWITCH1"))
 (segment (start 188.5603 101.05) (end 190.9603 93.45) (width 0.25) (layer "F.Cu") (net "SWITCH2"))
 (segment (start 190.9603 93.45) (end 193.5603 90.45) (width 0.25) (layer "F.Cu") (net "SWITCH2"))
 (segment (start 182.3603 120.25) (end 184.3603 112.85) (width 0.25) (layer "F.Cu") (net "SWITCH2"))
 (segment (start 193.5603 90.45) (end 195.9603 77.45) (width 0.25) (layer "F.Cu") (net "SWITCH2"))
 (segment (start 195.9603 58.05) (end 194.9603 56.85) (width 0.25) (layer "F.Cu") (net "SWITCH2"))
 (segment (start 195.9603 77.45) (end 195.9603 58.05) (width 0.25) (layer "F.Cu") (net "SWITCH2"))
 (segment (start 184.3603 112.85) (end 184.3603 110.25) (width 0.25) (layer "F.Cu") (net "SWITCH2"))
 (segment (start 184.3603 110.25) (end 188.5603 101.05) (width 0.25) (layer "F.Cu") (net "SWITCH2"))
 (segment (start 144.7603 87.65) (end 145.5603 87.05) (width 0.25) (layer "F.Cu") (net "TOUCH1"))
 (via (at 145.5603 87.05) (size 0.6) (drill 0.3) (layers "F.Cu" "B.Cu") (capping no) (covering (front no) (back no))
  (plugging (front no) (back no)) (filling no) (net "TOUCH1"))
 (segment (start 145.5603 87.05) (end 158.1603 79.45) (width 0.25) (layer "B.Cu") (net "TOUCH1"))
 (segment (start 158.1603 79.45) (end 178.7603 64.25) (width 0.25) (layer "B.Cu") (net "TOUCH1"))
 (segment (start 157.3603 66.45) (end 178.7603 66.45) (width 0.25) (layer "F.Cu") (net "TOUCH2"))
 (segment (start 164.5603 84.25) (end 178.9603 69.45) (width 0.25) (layer "F.Cu") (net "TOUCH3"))
 (segment (start 177.9603 73.25) (end 179.1603 72.05) (width 0.25) (layer "F.Cu") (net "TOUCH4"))
 (segment (start 170.1603 102.05) (end 171.1603 101.05) (width 0.25) (layer "F.Cu") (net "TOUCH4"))
 (segment (start 165.3603 104.85) (end 170.1603 102.05) (width 0.25) (layer "F.Cu") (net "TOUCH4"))
 (segment (start 157.3603 109.45) (end 165.3603 104.85) (width 0.25) (layer "F.Cu") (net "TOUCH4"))
 (segment (start 171.1603 101.05) (end 177.9603 73.25) (width 0.25) (layer "F.Cu") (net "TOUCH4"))
 (segment (start 132.1603 122.65) (end 133.5603 123.85) (width 0.25) (layer "F.Cu") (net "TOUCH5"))
 (segment (start 133.5603 123.85) (end 134.7603 124.65) (width 0.25) (layer "F.Cu") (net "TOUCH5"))
 (segment (start 180.7603 75.85) (end 179.5603 74.65) (width 0.25) (layer "F.Cu") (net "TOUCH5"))
 (segment (start 155.5603 125.65) (end 158.3603 123.05) (width 0.25) (layer "F.Cu") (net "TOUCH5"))
 (segment (start 146.3603 130.25) (end 155.5603 125.65) (width 0.25) (layer "F.Cu") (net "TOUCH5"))
 (segment (start 178.9603 90.45) (end 180.7603 77.25) (width 0.25) (layer "F.Cu") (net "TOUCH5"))
 (segment (start 180.7603 77.25) (end 180.7603 75.85) (width 0.25) (layer "F.Cu") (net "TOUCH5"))
 (segment (start 158.3603 123.05) (end 178.9603 90.45) (width 0.25) (layer "F.Cu") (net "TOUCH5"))
 (segment (start 144.5603 130.25) (end 146.3603 130.25) (width 0.25) (layer "F.Cu") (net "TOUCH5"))
 (segment (start 134.7603 124.65) (end 144.5603 130.25) (width 0.25) (layer "F.Cu") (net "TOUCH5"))
 (segment (start 165.5603 72.85) (end 170.7603 76.65) (width 0.25) (layer "F.Cu") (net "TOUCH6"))
 (segment (start 107.7603 80.85) (end 107.7603 79.45) (width 0.25) (layer "F.Cu") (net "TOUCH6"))
 (via (at 165.5603 72.85) (size 0.6) (drill 0.3) (layers "F.Cu" "B.Cu") (capping no) (covering (front no) (back no))
  (plugging (front no) (back no)) (filling no) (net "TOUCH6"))
 (via (at 107.7603 79.45) (size 0.6) (drill 0.3) (layers "F.Cu" "B.Cu") (capping no) (covering (front no) (back no))
  (plugging (front no) (back no)) (filling no) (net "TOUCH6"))
 (via (at 170.7603 76.65) (size 0.6) (drill 0.3) (layers "F.Cu" "B.Cu") (capping no) (covering (front no) (back no))
  (plugging (front no) (back no)) (filling no) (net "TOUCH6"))
 (segment (start 154.9603 63.05) (end 158.3603 65.65) (width 0.25) (layer "B.Cu") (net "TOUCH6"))
 (segment (start 170.7603 76.65) (end 178.7603 76.65) (width 0.25) (layer "B.Cu") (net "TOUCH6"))
 (segment (start 108.1603 65.05) (end 120.1603 58.25) (width 0.25) (layer "B.Cu") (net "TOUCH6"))
 (segment (start 146.9603 58.65) (end 154.9603 63.05) (width 0.25) (layer "B.Cu") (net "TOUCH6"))
 (segment (start 158.3603 65.65) (end 165.5603 72.85) (width 0.25) (layer "B.Cu") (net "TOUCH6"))
 (segment (start 120.1603 58.25) (end 146.9603 58.65) (width 0.25) (layer "B.Cu") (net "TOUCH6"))
 (segment (start 107.7603 79.45) (end 108.1603 65.05) (width 0.25) (layer "B.Cu") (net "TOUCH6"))
 (segment (start 132.1603 65.85) (end 133.5603 64.65) (width 0.25) (layer "F.Cu") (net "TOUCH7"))
 (segment (start 144.5603 58.25) (end 178.1603 54.85) (width 0.25) (layer "F.Cu") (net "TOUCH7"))
 (segment (start 193.3603 75.05) (end 194.1603 76.05) (width 0.25) (layer "F.Cu") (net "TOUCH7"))
 (segment (start 193.1603 74.65) (end 193.3603 75.05) (width 0.25) (layer "F.Cu") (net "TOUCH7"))
 (segment (start 192.5603 70.65) (end 193.1603 74.65) (width 0.25) (layer "F.Cu") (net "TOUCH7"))
 (segment (start 134.7603 63.85) (end 144.5603 58.25) (width 0.25) (layer "F.Cu") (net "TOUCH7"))
 (segment (start 180.5603 54.85) (end 192.5603 70.65) (width 0.25) (layer "F.Cu") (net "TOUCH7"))
 (segment (start 178.1603 54.85) (end 180.5603 54.85) (width 0.25) (layer "F.Cu") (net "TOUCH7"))
 (segment (start 133.5603 64.65) (end 134.7603 63.85) (width 0.25) (layer "F.Cu") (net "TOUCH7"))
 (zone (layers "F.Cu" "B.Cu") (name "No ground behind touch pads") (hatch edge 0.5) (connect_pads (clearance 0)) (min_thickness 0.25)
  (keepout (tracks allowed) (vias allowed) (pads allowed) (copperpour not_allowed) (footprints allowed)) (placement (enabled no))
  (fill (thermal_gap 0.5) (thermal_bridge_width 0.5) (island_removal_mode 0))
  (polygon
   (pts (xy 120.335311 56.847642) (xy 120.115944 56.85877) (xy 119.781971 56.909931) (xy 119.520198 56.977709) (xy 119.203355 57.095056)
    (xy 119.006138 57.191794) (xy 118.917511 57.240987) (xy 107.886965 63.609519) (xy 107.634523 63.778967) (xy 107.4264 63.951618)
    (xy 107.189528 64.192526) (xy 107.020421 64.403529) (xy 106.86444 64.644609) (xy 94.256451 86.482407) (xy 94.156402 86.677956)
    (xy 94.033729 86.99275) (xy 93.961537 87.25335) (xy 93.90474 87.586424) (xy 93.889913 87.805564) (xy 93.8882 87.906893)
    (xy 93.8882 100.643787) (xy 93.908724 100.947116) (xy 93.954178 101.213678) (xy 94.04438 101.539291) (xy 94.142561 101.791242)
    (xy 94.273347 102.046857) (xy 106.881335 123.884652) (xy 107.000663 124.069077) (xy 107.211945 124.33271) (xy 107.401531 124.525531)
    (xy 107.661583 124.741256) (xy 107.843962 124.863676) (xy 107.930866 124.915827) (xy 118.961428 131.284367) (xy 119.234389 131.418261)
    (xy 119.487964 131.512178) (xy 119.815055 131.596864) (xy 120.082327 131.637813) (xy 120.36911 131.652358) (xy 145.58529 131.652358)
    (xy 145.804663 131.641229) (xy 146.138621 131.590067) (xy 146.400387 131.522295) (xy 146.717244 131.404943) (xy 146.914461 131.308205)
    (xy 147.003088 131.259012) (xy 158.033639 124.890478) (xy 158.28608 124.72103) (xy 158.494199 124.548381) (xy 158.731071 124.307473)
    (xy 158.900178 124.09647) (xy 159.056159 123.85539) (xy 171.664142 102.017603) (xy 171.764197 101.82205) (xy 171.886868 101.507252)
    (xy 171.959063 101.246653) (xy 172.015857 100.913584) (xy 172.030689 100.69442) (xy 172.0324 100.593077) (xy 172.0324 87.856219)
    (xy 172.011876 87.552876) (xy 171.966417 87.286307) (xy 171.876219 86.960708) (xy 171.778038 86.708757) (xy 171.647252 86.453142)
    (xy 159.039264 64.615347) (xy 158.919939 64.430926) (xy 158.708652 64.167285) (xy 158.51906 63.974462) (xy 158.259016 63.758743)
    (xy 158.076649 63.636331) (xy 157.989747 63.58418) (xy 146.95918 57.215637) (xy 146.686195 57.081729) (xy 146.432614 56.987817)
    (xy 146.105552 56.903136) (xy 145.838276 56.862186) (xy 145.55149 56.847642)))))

